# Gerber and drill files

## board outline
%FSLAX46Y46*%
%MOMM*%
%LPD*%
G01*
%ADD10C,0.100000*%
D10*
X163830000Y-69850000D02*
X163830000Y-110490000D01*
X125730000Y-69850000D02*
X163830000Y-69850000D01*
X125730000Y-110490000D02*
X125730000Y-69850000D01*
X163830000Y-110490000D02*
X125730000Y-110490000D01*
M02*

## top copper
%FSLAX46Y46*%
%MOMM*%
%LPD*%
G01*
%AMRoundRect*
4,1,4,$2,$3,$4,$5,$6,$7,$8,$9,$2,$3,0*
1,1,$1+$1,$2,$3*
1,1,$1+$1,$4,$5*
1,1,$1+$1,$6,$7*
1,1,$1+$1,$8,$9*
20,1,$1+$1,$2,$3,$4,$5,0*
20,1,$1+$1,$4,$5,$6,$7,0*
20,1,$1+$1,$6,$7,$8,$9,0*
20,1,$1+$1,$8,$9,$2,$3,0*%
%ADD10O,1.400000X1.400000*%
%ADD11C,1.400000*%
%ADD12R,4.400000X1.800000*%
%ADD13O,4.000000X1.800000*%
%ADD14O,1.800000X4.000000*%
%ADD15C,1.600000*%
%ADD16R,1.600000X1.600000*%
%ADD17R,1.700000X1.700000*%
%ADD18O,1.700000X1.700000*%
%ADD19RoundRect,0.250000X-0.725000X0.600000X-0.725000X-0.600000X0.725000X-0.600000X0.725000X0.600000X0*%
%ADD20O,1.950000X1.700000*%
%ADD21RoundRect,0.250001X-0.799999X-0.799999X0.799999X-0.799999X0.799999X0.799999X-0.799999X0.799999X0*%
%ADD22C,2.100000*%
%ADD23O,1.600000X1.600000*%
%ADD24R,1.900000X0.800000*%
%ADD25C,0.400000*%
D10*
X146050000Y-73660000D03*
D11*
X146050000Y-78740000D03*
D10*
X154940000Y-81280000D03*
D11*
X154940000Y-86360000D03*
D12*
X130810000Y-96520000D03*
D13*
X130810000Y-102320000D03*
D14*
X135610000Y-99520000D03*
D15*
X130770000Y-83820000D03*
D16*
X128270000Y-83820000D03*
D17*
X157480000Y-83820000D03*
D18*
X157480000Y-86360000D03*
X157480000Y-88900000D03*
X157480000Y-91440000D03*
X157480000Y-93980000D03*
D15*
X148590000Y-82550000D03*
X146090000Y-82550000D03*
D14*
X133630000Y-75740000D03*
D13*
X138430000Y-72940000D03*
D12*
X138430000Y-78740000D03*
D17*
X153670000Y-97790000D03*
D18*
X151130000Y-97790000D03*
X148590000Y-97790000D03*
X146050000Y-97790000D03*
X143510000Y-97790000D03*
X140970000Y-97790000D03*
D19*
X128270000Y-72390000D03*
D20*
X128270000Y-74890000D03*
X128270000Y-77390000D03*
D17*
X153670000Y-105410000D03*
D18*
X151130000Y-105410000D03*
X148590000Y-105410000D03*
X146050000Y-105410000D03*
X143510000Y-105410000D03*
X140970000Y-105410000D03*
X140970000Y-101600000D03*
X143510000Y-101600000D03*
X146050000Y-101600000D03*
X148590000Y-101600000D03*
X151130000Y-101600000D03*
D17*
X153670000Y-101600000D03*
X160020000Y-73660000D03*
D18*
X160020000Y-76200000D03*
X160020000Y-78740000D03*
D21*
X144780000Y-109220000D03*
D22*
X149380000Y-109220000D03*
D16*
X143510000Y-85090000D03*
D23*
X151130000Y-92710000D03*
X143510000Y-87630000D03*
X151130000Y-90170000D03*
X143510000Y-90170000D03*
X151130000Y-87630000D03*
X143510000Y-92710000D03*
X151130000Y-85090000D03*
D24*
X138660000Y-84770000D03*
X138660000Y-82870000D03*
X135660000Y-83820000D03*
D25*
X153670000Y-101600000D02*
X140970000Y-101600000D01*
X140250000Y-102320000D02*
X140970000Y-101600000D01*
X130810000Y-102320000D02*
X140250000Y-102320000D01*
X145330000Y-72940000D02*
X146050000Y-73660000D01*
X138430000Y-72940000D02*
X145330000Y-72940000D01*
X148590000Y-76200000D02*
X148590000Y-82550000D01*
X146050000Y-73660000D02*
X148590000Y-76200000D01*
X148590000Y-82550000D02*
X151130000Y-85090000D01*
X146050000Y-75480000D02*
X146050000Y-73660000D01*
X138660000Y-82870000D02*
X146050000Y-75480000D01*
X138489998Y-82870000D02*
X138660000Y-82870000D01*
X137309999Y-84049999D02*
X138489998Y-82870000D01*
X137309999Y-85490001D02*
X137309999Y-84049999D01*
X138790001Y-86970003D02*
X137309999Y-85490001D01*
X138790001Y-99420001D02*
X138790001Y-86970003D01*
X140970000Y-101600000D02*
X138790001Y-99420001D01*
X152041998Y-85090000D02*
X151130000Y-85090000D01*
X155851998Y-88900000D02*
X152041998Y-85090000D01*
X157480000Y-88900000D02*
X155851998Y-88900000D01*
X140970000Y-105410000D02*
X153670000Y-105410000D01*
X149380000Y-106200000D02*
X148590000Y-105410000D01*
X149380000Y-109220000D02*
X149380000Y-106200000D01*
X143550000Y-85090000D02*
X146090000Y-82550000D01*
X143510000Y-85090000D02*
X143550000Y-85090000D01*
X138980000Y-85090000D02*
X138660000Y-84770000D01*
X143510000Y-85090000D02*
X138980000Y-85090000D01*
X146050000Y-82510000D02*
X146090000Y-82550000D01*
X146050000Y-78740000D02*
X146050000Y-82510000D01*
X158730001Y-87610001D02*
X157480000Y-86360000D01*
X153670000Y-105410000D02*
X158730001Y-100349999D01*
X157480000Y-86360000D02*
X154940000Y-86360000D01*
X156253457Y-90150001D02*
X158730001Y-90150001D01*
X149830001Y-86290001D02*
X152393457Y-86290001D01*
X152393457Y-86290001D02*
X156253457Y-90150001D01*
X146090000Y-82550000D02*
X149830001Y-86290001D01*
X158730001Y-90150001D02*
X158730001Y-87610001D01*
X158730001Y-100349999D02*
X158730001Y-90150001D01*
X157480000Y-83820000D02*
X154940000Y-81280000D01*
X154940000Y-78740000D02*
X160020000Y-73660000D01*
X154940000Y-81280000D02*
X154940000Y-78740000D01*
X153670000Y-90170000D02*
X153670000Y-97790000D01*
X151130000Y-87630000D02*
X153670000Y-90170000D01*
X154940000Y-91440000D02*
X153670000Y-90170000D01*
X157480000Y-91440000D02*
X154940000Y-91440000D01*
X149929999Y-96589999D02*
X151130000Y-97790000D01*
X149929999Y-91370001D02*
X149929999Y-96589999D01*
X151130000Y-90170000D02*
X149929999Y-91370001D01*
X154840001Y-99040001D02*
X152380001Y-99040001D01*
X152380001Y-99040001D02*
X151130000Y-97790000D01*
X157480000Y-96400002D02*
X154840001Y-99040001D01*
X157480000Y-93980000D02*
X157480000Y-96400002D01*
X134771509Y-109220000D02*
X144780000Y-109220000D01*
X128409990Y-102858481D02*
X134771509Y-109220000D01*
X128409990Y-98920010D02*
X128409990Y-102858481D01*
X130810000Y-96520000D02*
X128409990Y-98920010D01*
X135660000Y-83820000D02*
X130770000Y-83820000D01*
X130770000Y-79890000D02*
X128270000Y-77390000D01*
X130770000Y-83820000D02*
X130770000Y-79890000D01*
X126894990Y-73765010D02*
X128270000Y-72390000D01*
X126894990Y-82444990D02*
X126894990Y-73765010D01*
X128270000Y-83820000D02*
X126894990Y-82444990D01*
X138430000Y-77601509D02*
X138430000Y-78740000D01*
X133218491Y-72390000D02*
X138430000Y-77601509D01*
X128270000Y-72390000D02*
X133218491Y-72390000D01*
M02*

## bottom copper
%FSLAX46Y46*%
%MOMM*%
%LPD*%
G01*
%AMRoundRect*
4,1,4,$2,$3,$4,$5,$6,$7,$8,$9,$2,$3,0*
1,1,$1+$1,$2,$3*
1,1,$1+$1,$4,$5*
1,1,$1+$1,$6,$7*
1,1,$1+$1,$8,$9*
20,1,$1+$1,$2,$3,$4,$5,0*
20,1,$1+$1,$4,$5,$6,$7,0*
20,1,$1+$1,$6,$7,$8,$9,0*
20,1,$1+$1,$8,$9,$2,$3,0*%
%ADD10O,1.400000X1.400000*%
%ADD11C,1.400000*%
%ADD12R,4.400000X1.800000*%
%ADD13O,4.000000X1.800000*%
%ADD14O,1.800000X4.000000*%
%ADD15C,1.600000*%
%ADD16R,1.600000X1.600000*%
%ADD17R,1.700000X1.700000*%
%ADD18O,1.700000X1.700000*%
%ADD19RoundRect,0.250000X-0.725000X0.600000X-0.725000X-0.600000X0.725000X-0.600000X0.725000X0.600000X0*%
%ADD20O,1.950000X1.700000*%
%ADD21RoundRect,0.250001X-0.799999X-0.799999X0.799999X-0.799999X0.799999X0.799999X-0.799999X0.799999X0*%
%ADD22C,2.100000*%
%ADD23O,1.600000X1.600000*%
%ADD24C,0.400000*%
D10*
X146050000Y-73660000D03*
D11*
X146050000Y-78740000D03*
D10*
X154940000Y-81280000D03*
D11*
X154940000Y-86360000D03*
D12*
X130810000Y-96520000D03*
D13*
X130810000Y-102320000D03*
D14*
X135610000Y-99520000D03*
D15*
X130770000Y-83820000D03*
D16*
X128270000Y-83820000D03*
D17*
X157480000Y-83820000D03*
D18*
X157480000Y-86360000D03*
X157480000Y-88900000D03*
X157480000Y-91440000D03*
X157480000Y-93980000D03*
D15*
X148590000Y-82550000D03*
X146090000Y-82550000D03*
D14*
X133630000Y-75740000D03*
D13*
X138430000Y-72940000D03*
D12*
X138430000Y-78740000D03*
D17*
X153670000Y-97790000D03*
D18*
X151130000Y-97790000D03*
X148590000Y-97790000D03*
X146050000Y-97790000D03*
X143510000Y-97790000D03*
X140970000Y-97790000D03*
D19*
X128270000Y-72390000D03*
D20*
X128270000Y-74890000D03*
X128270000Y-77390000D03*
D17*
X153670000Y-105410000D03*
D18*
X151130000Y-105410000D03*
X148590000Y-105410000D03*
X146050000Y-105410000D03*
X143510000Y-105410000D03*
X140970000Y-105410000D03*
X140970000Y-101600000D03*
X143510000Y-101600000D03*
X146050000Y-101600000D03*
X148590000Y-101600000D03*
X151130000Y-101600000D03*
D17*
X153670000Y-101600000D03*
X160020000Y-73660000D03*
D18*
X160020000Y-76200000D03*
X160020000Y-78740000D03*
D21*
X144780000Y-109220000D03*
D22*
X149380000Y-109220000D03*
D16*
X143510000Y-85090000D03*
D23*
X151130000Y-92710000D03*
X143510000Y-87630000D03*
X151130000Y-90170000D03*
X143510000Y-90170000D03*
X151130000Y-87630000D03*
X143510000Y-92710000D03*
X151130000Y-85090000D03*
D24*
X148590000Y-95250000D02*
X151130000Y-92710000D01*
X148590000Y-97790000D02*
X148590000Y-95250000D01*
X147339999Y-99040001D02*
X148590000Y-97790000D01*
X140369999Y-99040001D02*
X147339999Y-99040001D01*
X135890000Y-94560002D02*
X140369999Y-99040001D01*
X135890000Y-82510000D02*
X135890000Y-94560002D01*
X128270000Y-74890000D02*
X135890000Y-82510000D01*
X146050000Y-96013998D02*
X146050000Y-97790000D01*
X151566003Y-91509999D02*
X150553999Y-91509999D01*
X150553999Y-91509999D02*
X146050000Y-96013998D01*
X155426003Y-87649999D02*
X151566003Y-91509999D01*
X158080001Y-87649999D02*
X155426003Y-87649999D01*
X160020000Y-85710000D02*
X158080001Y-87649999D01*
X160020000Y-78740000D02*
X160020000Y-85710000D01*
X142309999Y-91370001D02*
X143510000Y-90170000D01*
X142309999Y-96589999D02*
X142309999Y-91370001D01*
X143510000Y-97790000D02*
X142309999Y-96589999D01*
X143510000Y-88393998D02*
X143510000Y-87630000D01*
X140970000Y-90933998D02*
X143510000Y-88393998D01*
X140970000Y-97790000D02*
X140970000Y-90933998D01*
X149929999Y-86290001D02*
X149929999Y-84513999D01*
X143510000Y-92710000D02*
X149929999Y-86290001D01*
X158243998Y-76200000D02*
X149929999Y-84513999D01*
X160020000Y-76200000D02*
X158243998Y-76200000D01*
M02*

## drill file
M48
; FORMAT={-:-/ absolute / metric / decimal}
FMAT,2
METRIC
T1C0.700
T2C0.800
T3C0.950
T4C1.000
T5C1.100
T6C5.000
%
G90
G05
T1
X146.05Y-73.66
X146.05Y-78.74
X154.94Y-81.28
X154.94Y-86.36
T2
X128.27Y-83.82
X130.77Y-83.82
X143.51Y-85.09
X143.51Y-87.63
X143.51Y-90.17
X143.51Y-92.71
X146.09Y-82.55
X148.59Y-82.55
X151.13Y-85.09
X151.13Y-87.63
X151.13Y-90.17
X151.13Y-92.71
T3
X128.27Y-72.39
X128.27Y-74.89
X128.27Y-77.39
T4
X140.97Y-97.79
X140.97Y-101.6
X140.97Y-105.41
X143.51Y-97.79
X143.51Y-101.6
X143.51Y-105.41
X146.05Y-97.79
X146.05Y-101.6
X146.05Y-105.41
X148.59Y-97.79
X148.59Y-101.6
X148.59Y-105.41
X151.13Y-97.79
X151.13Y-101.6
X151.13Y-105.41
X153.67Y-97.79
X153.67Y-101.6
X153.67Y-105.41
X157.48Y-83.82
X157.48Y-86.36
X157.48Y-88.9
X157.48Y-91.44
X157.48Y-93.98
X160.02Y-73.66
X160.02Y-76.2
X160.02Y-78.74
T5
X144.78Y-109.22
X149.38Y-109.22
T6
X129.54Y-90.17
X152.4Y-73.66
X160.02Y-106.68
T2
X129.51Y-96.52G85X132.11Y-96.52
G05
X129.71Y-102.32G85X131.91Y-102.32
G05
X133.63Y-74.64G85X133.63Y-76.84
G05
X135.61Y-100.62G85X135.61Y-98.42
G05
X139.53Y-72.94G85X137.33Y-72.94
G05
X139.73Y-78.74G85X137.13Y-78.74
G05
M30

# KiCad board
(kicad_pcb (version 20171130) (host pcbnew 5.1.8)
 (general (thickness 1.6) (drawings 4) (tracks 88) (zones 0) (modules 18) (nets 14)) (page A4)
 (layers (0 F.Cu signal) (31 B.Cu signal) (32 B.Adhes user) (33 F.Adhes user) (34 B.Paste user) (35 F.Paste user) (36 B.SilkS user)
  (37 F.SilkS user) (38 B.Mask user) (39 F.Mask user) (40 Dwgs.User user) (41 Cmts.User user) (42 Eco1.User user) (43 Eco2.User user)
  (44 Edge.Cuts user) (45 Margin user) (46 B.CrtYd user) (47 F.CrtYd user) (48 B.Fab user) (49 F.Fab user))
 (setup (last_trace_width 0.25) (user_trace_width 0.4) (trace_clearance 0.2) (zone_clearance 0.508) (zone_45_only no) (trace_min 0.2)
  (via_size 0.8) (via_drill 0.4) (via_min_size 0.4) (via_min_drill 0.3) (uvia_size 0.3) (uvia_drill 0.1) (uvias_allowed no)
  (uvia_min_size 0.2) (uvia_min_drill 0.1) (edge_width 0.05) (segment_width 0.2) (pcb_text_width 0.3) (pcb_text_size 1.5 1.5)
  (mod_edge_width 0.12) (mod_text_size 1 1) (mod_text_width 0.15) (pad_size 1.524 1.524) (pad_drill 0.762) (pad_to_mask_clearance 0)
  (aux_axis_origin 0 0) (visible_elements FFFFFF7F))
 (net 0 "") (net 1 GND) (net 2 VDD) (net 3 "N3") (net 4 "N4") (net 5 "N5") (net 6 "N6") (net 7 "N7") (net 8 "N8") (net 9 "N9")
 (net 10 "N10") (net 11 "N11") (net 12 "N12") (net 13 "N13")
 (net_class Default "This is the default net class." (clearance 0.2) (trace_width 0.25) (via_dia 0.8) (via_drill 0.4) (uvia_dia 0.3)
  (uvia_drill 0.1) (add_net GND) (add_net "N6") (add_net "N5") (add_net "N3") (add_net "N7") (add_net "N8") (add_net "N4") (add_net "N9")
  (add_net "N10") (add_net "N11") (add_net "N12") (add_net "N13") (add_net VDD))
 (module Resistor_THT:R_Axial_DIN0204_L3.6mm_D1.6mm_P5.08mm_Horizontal (layer F.Cu) (at 146.05 78.74 90)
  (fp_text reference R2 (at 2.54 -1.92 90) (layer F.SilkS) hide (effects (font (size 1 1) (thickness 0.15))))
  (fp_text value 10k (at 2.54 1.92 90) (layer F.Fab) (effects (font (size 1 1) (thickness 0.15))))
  (pad 2 thru_hole oval (at 5.08 0 90) (size 1.4 1.4) (drill 0.7) (layers *.Cu *.Mask) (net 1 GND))
  (pad 1 thru_hole circle (at 0 0 90) (size 1.4 1.4) (drill 0.7) (layers *.Cu *.Mask) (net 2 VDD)))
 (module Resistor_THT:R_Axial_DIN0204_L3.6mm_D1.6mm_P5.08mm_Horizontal (layer F.Cu) (at 154.94 86.36 90)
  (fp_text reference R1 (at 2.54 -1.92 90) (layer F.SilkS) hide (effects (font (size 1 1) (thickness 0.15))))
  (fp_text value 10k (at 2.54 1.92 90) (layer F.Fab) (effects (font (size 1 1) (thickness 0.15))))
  (pad 2 thru_hole oval (at 5.08 0 90) (size 1.4 1.4) (drill 0.7) (layers *.Cu *.Mask) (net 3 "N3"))
  (pad 1 thru_hole circle (at 0 0 90) (size 1.4 1.4) (drill 0.7) (layers *.Cu *.Mask) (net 2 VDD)))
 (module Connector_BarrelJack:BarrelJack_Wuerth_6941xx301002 (layer F.Cu) (at 130.81 96.52)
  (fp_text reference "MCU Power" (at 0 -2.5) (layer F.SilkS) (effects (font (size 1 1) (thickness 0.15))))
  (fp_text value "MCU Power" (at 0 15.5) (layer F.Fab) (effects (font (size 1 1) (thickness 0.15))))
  (pad 1 thru_hole rect (at 0 0) (size 4.4 1.8) (drill oval 3.4 0.8) (layers *.Cu *.Mask) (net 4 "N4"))
  (pad 2 thru_hole oval (at 0 5.8) (size 4 1.8) (drill oval 3 0.8) (layers *.Cu *.Mask) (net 1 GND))
  (pad 3 thru_hole oval (at 4.8 3 90) (size 4 1.8) (drill oval 3 0.8) (layers *.Cu *.Mask)))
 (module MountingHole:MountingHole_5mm (layer F.Cu) (at 160.02 106.68)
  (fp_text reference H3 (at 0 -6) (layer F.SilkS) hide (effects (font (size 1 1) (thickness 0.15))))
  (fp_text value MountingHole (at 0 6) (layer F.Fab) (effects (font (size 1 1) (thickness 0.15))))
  (pad 1 np_thru_hole circle (at 0 0) (size 5 5) (drill 5) (layers *.Cu *.Mask)))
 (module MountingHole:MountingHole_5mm (layer F.Cu) (at 129.54 90.17)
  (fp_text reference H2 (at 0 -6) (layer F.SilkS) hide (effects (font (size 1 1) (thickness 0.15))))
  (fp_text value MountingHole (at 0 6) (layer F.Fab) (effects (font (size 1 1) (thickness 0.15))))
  (pad 1 np_thru_hole circle (at 0 0) (size 5 5) (drill 5) (layers *.Cu *.Mask)))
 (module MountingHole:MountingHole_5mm (layer F.Cu) (at 152.4 73.66)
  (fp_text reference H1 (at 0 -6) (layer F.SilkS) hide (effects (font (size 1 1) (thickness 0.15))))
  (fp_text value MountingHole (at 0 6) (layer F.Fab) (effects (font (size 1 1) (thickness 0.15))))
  (pad 1 np_thru_hole circle (at 0 0) (size 5 5) (drill 5) (layers *.Cu *.Mask)))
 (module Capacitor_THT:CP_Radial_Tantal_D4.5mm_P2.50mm (layer F.Cu) (at 128.27 83.82)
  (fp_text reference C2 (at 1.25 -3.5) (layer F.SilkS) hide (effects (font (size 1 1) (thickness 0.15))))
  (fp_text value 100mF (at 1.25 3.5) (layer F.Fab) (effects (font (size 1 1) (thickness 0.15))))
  (pad 2 thru_hole circle (at 2.5 0) (size 1.6 1.6) (drill 0.8) (layers *.Cu *.Mask) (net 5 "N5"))
  (pad 1 thru_hole rect (at 0 0) (size 1.6 1.6) (drill 0.8) (layers *.Cu *.Mask) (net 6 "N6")))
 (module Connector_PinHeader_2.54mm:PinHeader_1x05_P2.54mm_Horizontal (layer F.Cu) (at 157.48 83.82)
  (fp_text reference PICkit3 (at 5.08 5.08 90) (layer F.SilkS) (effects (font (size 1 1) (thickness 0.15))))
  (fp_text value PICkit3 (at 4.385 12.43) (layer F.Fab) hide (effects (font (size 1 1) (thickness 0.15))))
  (pad 1 thru_hole rect (at 0 0) (size 1.7 1.7) (drill 1) (layers *.Cu *.Mask) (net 3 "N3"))
  (pad 2 thru_hole oval (at 0 2.54) (size 1.7 1.7) (drill 1) (layers *.Cu *.Mask) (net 2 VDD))
  (pad 3 thru_hole oval (at 0 5.08) (size 1.7 1.7) (drill 1) (layers *.Cu *.Mask) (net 1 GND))
  (pad 4 thru_hole oval (at 0 7.62) (size 1.7 1.7) (drill 1) (layers *.Cu *.Mask) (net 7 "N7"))
  (pad 5 thru_hole oval (at 0 10.16) (size 1.7 1.7) (drill 1) (layers *.Cu *.Mask) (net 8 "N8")))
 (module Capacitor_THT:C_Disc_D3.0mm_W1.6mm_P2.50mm (layer F.Cu) (at 148.59 82.55 180)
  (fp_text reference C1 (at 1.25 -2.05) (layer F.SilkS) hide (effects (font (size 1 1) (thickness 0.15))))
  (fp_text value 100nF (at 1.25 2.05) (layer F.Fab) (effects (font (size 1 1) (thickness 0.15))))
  (pad 1 thru_hole circle (at 0 0 180) (size 1.6 1.6) (drill 0.8) (layers *.Cu *.Mask) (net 1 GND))
  (pad 2 thru_hole circle (at 2.5 0 180) (size 1.6 1.6) (drill 0.8) (layers *.Cu *.Mask) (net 2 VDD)))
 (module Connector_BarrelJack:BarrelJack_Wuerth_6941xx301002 (layer F.Cu) (at 138.43 78.74 180)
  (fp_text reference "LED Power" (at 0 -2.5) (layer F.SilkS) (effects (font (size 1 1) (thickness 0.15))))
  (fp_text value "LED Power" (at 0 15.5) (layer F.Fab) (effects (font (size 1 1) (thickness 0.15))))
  (pad 3 thru_hole oval (at 4.8 3 270) (size 4 1.8) (drill oval 3 0.8) (layers *.Cu *.Mask))
  (pad 2 thru_hole oval (at 0 5.8 180) (size 4 1.8) (drill oval 3 0.8) (layers *.Cu *.Mask) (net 1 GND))
  (pad 1 thru_hole rect (at 0 0 180) (size 4.4 1.8) (drill oval 3.4 0.8) (layers *.Cu *.Mask) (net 6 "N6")))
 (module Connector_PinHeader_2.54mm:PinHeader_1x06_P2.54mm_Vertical (layer F.Cu) (at 153.67 97.79 270)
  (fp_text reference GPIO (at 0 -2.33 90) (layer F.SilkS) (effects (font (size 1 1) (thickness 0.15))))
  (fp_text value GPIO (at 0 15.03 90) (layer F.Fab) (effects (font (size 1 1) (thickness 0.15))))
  (pad 1 thru_hole rect (at 0 0 270) (size 1.7 1.7) (drill 1) (layers *.Cu *.Mask) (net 7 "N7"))
  (pad 2 thru_hole oval (at 0 2.54 270) (size 1.7 1.7) (drill 1) (layers *.Cu *.Mask) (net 8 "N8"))
  (pad 3 thru_hole oval (at 0 5.08 270) (size 1.7 1.7) (drill 1) (layers *.Cu *.Mask) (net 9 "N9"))
  (pad 4 thru_hole oval (at 0 7.62 270) (size 1.7 1.7) (drill 1) (layers *.Cu *.Mask) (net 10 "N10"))
  (pad 5 thru_hole oval (at 0 10.16 270) (size 1.7 1.7) (drill 1) (layers *.Cu *.Mask) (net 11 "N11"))
  (pad 6 thru_hole oval (at 0 12.7 270) (size 1.7 1.7) (drill 1) (layers *.Cu *.Mask) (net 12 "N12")))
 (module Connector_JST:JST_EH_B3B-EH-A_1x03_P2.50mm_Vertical (layer F.Cu) (at 128.27 72.39 270)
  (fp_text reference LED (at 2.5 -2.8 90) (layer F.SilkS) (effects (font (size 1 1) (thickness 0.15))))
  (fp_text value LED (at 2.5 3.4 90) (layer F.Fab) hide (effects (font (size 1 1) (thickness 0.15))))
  (pad 1 thru_hole roundrect (at 0 0 270) (size 1.7 1.95) (drill 0.95) (layers *.Cu *.Mask) (roundrect_rratio 0.147059) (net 6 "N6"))
  (pad 2 thru_hole oval (at 2.5 0 270) (size 1.7 1.95) (drill 0.95) (layers *.Cu *.Mask) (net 9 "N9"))
  (pad 3 thru_hole oval (at 5 0 270) (size 1.7 1.95) (drill 0.95) (layers *.Cu *.Mask) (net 5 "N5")))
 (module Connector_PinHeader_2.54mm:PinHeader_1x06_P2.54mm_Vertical (layer F.Cu) (at 153.67 105.41 270)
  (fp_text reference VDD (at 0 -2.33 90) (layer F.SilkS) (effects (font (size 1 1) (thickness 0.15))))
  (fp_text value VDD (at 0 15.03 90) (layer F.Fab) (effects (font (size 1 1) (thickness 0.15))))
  (pad 1 thru_hole rect (at 0 0 270) (size 1.7 1.7) (drill 1) (layers *.Cu *.Mask) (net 2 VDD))
  (pad 2 thru_hole oval (at 0 2.54 270) (size 1.7 1.7) (drill 1) (layers *.Cu *.Mask) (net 2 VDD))
  (pad 3 thru_hole oval (at 0 5.08 270) (size 1.7 1.7) (drill 1) (layers *.Cu *.Mask) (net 2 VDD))
  (pad 4 thru_hole oval (at 0 7.62 270) (size 1.7 1.7) (drill 1) (layers *.Cu *.Mask) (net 2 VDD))
  (pad 5 thru_hole oval (at 0 10.16 270) (size 1.7 1.7) (drill 1) (layers *.Cu *.Mask) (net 2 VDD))
  (pad 6 thru_hole oval (at 0 12.7 270) (size 1.7 1.7) (drill 1) (layers *.Cu *.Mask) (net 2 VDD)))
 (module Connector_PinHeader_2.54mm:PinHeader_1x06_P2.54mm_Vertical (layer F.Cu) (at 153.67 101.6 270)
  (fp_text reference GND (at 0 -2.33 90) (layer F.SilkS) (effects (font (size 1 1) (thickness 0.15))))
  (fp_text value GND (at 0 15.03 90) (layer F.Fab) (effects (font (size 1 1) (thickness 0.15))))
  (pad 6 thru_hole oval (at 0 12.7 270) (size 1.7 1.7) (drill 1) (layers *.Cu *.Mask) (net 1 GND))
  (pad 5 thru_hole oval (at 0 10.16 270) (size 1.7 1.7) (drill 1) (layers *.Cu *.Mask) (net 1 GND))
  (pad 4 thru_hole oval (at 0 7.62 270) (size 1.7 1.7) (drill 1) (layers *.Cu *.Mask) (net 1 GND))
  (pad 3 thru_hole oval (at 0 5.08 270) (size 1.7 1.7) (drill 1) (layers *.Cu *.Mask) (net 1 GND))
  (pad 2 thru_hole oval (at 0 2.54 270) (size 1.7 1.7) (drill 1) (layers *.Cu *.Mask) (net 1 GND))
  (pad 1 thru_hole rect (at 0 0 270) (size 1.7 1.7) (drill 1) (layers *.Cu *.Mask) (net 1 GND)))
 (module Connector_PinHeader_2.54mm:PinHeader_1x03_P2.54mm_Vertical (layer F.Cu) (at 160.02 73.66)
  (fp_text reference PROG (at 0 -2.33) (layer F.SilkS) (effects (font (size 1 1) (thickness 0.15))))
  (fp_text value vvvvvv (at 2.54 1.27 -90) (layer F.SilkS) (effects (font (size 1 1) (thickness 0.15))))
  (pad 1 thru_hole rect (at 0 0) (size 1.7 1.7) (drill 1) (layers *.Cu *.Mask) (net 3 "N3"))
  (pad 2 thru_hole oval (at 0 2.54) (size 1.7 1.7) (drill 1) (layers *.Cu *.Mask) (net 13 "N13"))
  (pad 3 thru_hole oval (at 0 5.08) (size 1.7 1.7) (drill 1) (layers *.Cu *.Mask) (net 10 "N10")))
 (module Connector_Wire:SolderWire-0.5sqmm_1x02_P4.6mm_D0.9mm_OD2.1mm (layer F.Cu) (at 144.78 109.22)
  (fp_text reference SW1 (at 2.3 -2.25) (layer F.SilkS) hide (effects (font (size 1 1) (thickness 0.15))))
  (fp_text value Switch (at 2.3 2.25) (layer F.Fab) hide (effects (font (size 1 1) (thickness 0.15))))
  (pad 1 thru_hole roundrect (at 0 0) (size 2.1 2.1) (drill 1.1) (layers *.Cu *.Mask) (roundrect_rratio 0.119048) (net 4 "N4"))
  (pad 2 thru_hole circle (at 4.6 0) (size 2.1 2.1) (drill 1.1) (layers *.Cu *.Mask) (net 2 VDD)))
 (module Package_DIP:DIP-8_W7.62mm (layer F.Cu) (at 143.51 85.09)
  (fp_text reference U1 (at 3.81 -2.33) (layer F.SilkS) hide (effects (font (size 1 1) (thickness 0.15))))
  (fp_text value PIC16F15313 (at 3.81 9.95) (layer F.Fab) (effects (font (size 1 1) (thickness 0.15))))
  (pad 1 thru_hole rect (at 0 0) (size 1.6 1.6) (drill 0.8) (layers *.Cu *.Mask) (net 2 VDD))
  (pad 5 thru_hole oval (at 7.62 7.62) (size 1.6 1.6) (drill 0.8) (layers *.Cu *.Mask) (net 9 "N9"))
  (pad 2 thru_hole oval (at 0 2.54) (size 1.6 1.6) (drill 0.8) (layers *.Cu *.Mask) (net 12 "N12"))
  (pad 6 thru_hole oval (at 7.62 5.08) (size 1.6 1.6) (drill 0.8) (layers *.Cu *.Mask) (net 8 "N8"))
  (pad 3 thru_hole oval (at 0 5.08) (size 1.6 1.6) (drill 0.8) (layers *.Cu *.Mask) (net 11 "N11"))
  (pad 7 thru_hole oval (at 7.62 2.54) (size 1.6 1.6) (drill 0.8) (layers *.Cu *.Mask) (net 7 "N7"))
  (pad 4 thru_hole oval (at 0 7.62) (size 1.6 1.6) (drill 0.8) (layers *.Cu *.Mask) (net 13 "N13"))
  (pad 8 thru_hole oval (at 7.62 0) (size 1.6 1.6) (drill 0.8) (layers *.Cu *.Mask) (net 1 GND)))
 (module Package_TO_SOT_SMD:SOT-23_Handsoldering (layer F.Cu) (at 137.16 83.82 180)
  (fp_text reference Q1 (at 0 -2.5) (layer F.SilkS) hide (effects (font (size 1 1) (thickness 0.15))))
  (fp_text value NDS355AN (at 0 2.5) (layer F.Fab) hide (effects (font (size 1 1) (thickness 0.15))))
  (pad 1 smd rect (at -1.5 -0.95 180) (size 1.9 0.8) (layers F.Cu F.Paste F.Mask) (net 2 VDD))
  (pad 2 smd rect (at -1.5 0.95 180) (size 1.9 0.8) (layers F.Cu F.Paste F.Mask) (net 1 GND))
  (pad 3 smd rect (at 1.5 0 180) (size 1.9 0.8) (layers F.Cu F.Paste F.Mask) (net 5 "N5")))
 (gr_line (start 163.83 69.85) (end 163.83 110.49) (layer Edge.Cuts) (width 0.1))
 (gr_line (start 125.73 69.85) (end 163.83 69.85) (layer Edge.Cuts) (width 0.1))
 (gr_line (start 125.73 110.49) (end 125.73 69.85) (layer Edge.Cuts) (width 0.1))
 (gr_line (start 163.83 110.49) (end 125.73 110.49) (layer Edge.Cuts) (width 0.1))
 (segment (start 153.67 101.6) (end 140.97 101.6) (width 0.4) (layer F.Cu) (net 1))
 (segment (start 140.25 102.32) (end 140.97 101.6) (width 0.4) (layer F.Cu) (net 1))
 (segment (start 130.81 102.32) (end 140.25 102.32) (width 0.4) (layer F.Cu) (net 1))
 (segment (start 145.33 72.94) (end 146.05 73.66) (width 0.4) (layer F.Cu) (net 1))
 (segment (start 138.43 72.94) (end 145.33 72.94) (width 0.4) (layer F.Cu) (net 1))
 (segment (start 148.59 76.2) (end 148.59 82.55) (width 0.4) (layer F.Cu) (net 1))
 (segment (start 146.05 73.66) (end 148.59 76.2) (width 0.4) (layer F.Cu) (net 1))
 (segment (start 148.59 82.55) (end 151.13 85.09) (width 0.4) (layer F.Cu) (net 1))
 (segment (start 146.05 75.48) (end 146.05 73.66) (width 0.4) (layer F.Cu) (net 1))
 (segment (start 138.66 82.87) (end 146.05 75.48) (width 0.4) (layer F.Cu) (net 1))
 (segment (start 138.489998 82.87) (end 138.66 82.87) (width 0.4) (layer F.Cu) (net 1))
 (segment (start 137.309999 84.049999) (end 138.489998 82.87) (width 0.4) (layer F.Cu) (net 1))
 (segment (start 137.309999 85.490001) (end 137.309999 84.049999) (width 0.4) (layer F.Cu) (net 1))
 (segment (start 138.790001 86.970003) (end 137.309999 85.490001) (width 0.4) (layer F.Cu) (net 1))
 (segment (start 138.790001 99.420001) (end 138.790001 86.970003) (width 0.4) (layer F.Cu) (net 1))
 (segment (start 140.97 101.6) (end 138.790001 99.420001) (width 0.4) (layer F.Cu) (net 1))
 (segment (start 152.041998 85.09) (end 151.13 85.09) (width 0.4) (layer F.Cu) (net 1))
 (segment (start 155.851998 88.9) (end 152.041998 85.09) (width 0.4) (layer F.Cu) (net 1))
 (segment (start 157.48 88.9) (end 155.851998 88.9) (width 0.4) (layer F.Cu) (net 1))
 (segment (start 140.97 105.41) (end 153.67 105.41) (width 0.4) (layer F.Cu) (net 2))
 (segment (start 149.38 106.2) (end 148.59 105.41) (width 0.4) (layer F.Cu) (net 2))
 (segment (start 149.38 109.22) (end 149.38 106.2) (width 0.4) (layer F.Cu) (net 2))
 (segment (start 143.55 85.09) (end 146.09 82.55) (width 0.4) (layer F.Cu) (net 2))
 (segment (start 143.51 85.09) (end 143.55 85.09) (width 0.4) (layer F.Cu) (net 2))
 (segment (start 138.98 85.09) (end 138.66 84.77) (width 0.4) (layer F.Cu) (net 2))
 (segment (start 143.51 85.09) (end 138.98 85.09) (width 0.4) (layer F.Cu) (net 2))
 (segment (start 146.05 82.51) (end 146.09 82.55) (width 0.4) (layer F.Cu) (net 2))
 (segment (start 146.05 78.74) (end 146.05 82.51) (width 0.4) (layer F.Cu) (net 2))
 (segment (start 158.730001 87.610001) (end 157.48 86.36) (width 0.4) (layer F.Cu) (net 2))
 (segment (start 153.67 105.41) (end 158.730001 100.349999) (width 0.4) (layer F.Cu) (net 2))
 (segment (start 157.48 86.36) (end 154.94 86.36) (width 0.4) (layer F.Cu) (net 2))
 (segment (start 156.253457 90.150001) (end 158.730001 90.150001) (width 0.4) (layer F.Cu) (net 2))
 (segment (start 149.830001 86.290001) (end 152.393457 86.290001) (width 0.4) (layer F.Cu) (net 2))
 (segment (start 152.393457 86.290001) (end 156.253457 90.150001) (width 0.4) (layer F.Cu) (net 2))
 (segment (start 146.09 82.55) (end 149.830001 86.290001) (width 0.4) (layer F.Cu) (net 2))
 (segment (start 158.730001 90.150001) (end 158.730001 87.610001) (width 0.4) (layer F.Cu) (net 2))
 (segment (start 158.730001 100.349999) (end 158.730001 90.150001) (width 0.4) (layer F.Cu) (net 2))
 (segment (start 157.48 83.82) (end 154.94 81.28) (width 0.4) (layer F.Cu) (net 3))
 (segment (start 154.94 78.74) (end 160.02 73.66) (width 0.4) (layer F.Cu) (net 3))
 (segment (start 154.94 81.28) (end 154.94 78.74) (width 0.4) (layer F.Cu) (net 3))
 (segment (start 153.67 90.17) (end 153.67 97.79) (width 0.4) (layer F.Cu) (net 7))
 (segment (start 151.13 87.63) (end 153.67 90.17) (width 0.4) (layer F.Cu) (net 7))
 (segment (start 154.94 91.44) (end 153.67 90.17) (width 0.4) (layer F.Cu) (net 7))
 (segment (start 157.48 91.44) (end 154.94 91.44) (width 0.4) (layer F.Cu) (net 7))
 (segment (start 149.929999 96.589999) (end 151.13 97.79) (width 0.4) (layer F.Cu) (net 8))
 (segment (start 149.929999 91.370001) (end 149.929999 96.589999) (width 0.4) (layer F.Cu) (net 8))
 (segment (start 151.13 90.17) (end 149.929999 91.370001) (width 0.4) (layer F.Cu) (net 8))
 (segment (start 154.840001 99.040001) (end 152.380001 99.040001) (width 0.4) (layer F.Cu) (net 8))
 (segment (start 152.380001 99.040001) (end 151.13 97.79) (width 0.4) (layer F.Cu) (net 8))
 (segment (start 157.48 96.400002) (end 154.840001 99.040001) (width 0.4) (layer F.Cu) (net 8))
 (segment (start 157.48 93.98) (end 157.48 96.400002) (width 0.4) (layer F.Cu) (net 8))
 (segment (start 134.771509 109.22) (end 144.78 109.22) (width 0.4) (layer F.Cu) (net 4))
 (segment (start 128.40999 102.858481) (end 134.771509 109.22) (width 0.4) (layer F.Cu) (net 4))
 (segment (start 128.40999 98.92001) (end 128.40999 102.858481) (width 0.4) (layer F.Cu) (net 4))
 (segment (start 130.81 96.52) (end 128.40999 98.92001) (width 0.4) (layer F.Cu) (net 4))
 (segment (start 148.59 95.25) (end 151.13 92.71) (width 0.4) (layer B.Cu) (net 9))
 (segment (start 148.59 97.79) (end 148.59 95.25) (width 0.4) (layer B.Cu) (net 9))
 (segment (start 147.339999 99.040001) (end 148.59 97.79) (width 0.4) (layer B.Cu) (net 9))
 (segment (start 140.369999 99.040001) (end 147.339999 99.040001) (width 0.4) (layer B.Cu) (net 9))
 (segment (start 135.89 94.560002) (end 140.369999 99.040001) (width 0.4) (layer B.Cu) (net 9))
 (segment (start 135.89 82.51) (end 135.89 94.560002) (width 0.4) (layer B.Cu) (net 9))
 (segment (start 128.27 74.89) (end 135.89 82.51) (width 0.4) (layer B.Cu) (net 9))
 (segment (start 146.05 96.013998) (end 146.05 97.79) (width 0.4) (layer B.Cu) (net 10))
 (segment (start 151.566003 91.509999) (end 150.553999 91.509999) (width 0.4) (layer B.Cu) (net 10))
 (segment (start 150.553999 91.509999) (end 146.05 96.013998) (width 0.4) (layer B.Cu) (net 10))
 (segment (start 155.426003 87.649999) (end 151.566003 91.509999) (width 0.4) (layer B.Cu) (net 10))
 (segment (start 158.080001 87.649999) (end 155.426003 87.649999) (width 0.4) (layer B.Cu) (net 10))
 (segment (start 160.02 85.71) (end 158.080001 87.649999) (width 0.4) (layer B.Cu) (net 10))
 (segment (start 160.02 78.74) (end 160.02 85.71) (width 0.4) (layer B.Cu) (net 10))
 (segment (start 142.309999 91.370001) (end 143.51 90.17) (width 0.4) (layer B.Cu) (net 11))
 (segment (start 142.309999 96.589999) (end 142.309999 91.370001) (width 0.4) (layer B.Cu) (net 11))
 (segment (start 143.51 97.79) (end 142.309999 96.589999) (width 0.4) (layer B.Cu) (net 11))
 (segment (start 143.51 88.393998) (end 143.51 87.63) (width 0.4) (layer B.Cu) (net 12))
 (segment (start 140.97 90.933998) (end 143.51 88.393998) (width 0.4) (layer B.Cu) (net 12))
 (segment (start 140.97 97.79) (end 140.97 90.933998) (width 0.4) (layer B.Cu) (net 12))
 (segment (start 149.929999 86.290001) (end 149.929999 84.513999) (width 0.4) (layer B.Cu) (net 13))
 (segment (start 143.51 92.71) (end 149.929999 86.290001) (width 0.4) (layer B.Cu) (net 13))
 (segment (start 158.243998 76.2) (end 149.929999 84.513999) (width 0.4) (layer B.Cu) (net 13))
 (segment (start 160.02 76.2) (end 158.243998 76.2) (width 0.4) (layer B.Cu) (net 13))
 (segment (start 135.66 83.82) (end 130.77 83.82) (width 0.4) (layer F.Cu) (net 5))
 (segment (start 130.77 79.89) (end 128.27 77.39) (width 0.4) (layer F.Cu) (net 5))
 (segment (start 130.77 83.82) (end 130.77 79.89) (width 0.4) (layer F.Cu) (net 5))
 (segment (start 126.89499 73.76501) (end 128.27 72.39) (width 0.4) (layer F.Cu) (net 6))
 (segment (start 126.89499 82.44499) (end 126.89499 73.76501) (width 0.4) (layer F.Cu) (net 6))
 (segment (start 128.27 83.82) (end 126.89499 82.44499) (width 0.4) (layer F.Cu) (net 6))
 (segment (start 138.43 77.601509) (end 138.43 78.74) (width 0.4) (layer F.Cu) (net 6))
 (segment (start 133.218491 72.39) (end 138.43 77.601509) (width 0.4) (layer F.Cu) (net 6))
 (segment (start 128.27 72.39) (end 133.218491 72.39) (width 0.4) (layer F.Cu) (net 6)))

